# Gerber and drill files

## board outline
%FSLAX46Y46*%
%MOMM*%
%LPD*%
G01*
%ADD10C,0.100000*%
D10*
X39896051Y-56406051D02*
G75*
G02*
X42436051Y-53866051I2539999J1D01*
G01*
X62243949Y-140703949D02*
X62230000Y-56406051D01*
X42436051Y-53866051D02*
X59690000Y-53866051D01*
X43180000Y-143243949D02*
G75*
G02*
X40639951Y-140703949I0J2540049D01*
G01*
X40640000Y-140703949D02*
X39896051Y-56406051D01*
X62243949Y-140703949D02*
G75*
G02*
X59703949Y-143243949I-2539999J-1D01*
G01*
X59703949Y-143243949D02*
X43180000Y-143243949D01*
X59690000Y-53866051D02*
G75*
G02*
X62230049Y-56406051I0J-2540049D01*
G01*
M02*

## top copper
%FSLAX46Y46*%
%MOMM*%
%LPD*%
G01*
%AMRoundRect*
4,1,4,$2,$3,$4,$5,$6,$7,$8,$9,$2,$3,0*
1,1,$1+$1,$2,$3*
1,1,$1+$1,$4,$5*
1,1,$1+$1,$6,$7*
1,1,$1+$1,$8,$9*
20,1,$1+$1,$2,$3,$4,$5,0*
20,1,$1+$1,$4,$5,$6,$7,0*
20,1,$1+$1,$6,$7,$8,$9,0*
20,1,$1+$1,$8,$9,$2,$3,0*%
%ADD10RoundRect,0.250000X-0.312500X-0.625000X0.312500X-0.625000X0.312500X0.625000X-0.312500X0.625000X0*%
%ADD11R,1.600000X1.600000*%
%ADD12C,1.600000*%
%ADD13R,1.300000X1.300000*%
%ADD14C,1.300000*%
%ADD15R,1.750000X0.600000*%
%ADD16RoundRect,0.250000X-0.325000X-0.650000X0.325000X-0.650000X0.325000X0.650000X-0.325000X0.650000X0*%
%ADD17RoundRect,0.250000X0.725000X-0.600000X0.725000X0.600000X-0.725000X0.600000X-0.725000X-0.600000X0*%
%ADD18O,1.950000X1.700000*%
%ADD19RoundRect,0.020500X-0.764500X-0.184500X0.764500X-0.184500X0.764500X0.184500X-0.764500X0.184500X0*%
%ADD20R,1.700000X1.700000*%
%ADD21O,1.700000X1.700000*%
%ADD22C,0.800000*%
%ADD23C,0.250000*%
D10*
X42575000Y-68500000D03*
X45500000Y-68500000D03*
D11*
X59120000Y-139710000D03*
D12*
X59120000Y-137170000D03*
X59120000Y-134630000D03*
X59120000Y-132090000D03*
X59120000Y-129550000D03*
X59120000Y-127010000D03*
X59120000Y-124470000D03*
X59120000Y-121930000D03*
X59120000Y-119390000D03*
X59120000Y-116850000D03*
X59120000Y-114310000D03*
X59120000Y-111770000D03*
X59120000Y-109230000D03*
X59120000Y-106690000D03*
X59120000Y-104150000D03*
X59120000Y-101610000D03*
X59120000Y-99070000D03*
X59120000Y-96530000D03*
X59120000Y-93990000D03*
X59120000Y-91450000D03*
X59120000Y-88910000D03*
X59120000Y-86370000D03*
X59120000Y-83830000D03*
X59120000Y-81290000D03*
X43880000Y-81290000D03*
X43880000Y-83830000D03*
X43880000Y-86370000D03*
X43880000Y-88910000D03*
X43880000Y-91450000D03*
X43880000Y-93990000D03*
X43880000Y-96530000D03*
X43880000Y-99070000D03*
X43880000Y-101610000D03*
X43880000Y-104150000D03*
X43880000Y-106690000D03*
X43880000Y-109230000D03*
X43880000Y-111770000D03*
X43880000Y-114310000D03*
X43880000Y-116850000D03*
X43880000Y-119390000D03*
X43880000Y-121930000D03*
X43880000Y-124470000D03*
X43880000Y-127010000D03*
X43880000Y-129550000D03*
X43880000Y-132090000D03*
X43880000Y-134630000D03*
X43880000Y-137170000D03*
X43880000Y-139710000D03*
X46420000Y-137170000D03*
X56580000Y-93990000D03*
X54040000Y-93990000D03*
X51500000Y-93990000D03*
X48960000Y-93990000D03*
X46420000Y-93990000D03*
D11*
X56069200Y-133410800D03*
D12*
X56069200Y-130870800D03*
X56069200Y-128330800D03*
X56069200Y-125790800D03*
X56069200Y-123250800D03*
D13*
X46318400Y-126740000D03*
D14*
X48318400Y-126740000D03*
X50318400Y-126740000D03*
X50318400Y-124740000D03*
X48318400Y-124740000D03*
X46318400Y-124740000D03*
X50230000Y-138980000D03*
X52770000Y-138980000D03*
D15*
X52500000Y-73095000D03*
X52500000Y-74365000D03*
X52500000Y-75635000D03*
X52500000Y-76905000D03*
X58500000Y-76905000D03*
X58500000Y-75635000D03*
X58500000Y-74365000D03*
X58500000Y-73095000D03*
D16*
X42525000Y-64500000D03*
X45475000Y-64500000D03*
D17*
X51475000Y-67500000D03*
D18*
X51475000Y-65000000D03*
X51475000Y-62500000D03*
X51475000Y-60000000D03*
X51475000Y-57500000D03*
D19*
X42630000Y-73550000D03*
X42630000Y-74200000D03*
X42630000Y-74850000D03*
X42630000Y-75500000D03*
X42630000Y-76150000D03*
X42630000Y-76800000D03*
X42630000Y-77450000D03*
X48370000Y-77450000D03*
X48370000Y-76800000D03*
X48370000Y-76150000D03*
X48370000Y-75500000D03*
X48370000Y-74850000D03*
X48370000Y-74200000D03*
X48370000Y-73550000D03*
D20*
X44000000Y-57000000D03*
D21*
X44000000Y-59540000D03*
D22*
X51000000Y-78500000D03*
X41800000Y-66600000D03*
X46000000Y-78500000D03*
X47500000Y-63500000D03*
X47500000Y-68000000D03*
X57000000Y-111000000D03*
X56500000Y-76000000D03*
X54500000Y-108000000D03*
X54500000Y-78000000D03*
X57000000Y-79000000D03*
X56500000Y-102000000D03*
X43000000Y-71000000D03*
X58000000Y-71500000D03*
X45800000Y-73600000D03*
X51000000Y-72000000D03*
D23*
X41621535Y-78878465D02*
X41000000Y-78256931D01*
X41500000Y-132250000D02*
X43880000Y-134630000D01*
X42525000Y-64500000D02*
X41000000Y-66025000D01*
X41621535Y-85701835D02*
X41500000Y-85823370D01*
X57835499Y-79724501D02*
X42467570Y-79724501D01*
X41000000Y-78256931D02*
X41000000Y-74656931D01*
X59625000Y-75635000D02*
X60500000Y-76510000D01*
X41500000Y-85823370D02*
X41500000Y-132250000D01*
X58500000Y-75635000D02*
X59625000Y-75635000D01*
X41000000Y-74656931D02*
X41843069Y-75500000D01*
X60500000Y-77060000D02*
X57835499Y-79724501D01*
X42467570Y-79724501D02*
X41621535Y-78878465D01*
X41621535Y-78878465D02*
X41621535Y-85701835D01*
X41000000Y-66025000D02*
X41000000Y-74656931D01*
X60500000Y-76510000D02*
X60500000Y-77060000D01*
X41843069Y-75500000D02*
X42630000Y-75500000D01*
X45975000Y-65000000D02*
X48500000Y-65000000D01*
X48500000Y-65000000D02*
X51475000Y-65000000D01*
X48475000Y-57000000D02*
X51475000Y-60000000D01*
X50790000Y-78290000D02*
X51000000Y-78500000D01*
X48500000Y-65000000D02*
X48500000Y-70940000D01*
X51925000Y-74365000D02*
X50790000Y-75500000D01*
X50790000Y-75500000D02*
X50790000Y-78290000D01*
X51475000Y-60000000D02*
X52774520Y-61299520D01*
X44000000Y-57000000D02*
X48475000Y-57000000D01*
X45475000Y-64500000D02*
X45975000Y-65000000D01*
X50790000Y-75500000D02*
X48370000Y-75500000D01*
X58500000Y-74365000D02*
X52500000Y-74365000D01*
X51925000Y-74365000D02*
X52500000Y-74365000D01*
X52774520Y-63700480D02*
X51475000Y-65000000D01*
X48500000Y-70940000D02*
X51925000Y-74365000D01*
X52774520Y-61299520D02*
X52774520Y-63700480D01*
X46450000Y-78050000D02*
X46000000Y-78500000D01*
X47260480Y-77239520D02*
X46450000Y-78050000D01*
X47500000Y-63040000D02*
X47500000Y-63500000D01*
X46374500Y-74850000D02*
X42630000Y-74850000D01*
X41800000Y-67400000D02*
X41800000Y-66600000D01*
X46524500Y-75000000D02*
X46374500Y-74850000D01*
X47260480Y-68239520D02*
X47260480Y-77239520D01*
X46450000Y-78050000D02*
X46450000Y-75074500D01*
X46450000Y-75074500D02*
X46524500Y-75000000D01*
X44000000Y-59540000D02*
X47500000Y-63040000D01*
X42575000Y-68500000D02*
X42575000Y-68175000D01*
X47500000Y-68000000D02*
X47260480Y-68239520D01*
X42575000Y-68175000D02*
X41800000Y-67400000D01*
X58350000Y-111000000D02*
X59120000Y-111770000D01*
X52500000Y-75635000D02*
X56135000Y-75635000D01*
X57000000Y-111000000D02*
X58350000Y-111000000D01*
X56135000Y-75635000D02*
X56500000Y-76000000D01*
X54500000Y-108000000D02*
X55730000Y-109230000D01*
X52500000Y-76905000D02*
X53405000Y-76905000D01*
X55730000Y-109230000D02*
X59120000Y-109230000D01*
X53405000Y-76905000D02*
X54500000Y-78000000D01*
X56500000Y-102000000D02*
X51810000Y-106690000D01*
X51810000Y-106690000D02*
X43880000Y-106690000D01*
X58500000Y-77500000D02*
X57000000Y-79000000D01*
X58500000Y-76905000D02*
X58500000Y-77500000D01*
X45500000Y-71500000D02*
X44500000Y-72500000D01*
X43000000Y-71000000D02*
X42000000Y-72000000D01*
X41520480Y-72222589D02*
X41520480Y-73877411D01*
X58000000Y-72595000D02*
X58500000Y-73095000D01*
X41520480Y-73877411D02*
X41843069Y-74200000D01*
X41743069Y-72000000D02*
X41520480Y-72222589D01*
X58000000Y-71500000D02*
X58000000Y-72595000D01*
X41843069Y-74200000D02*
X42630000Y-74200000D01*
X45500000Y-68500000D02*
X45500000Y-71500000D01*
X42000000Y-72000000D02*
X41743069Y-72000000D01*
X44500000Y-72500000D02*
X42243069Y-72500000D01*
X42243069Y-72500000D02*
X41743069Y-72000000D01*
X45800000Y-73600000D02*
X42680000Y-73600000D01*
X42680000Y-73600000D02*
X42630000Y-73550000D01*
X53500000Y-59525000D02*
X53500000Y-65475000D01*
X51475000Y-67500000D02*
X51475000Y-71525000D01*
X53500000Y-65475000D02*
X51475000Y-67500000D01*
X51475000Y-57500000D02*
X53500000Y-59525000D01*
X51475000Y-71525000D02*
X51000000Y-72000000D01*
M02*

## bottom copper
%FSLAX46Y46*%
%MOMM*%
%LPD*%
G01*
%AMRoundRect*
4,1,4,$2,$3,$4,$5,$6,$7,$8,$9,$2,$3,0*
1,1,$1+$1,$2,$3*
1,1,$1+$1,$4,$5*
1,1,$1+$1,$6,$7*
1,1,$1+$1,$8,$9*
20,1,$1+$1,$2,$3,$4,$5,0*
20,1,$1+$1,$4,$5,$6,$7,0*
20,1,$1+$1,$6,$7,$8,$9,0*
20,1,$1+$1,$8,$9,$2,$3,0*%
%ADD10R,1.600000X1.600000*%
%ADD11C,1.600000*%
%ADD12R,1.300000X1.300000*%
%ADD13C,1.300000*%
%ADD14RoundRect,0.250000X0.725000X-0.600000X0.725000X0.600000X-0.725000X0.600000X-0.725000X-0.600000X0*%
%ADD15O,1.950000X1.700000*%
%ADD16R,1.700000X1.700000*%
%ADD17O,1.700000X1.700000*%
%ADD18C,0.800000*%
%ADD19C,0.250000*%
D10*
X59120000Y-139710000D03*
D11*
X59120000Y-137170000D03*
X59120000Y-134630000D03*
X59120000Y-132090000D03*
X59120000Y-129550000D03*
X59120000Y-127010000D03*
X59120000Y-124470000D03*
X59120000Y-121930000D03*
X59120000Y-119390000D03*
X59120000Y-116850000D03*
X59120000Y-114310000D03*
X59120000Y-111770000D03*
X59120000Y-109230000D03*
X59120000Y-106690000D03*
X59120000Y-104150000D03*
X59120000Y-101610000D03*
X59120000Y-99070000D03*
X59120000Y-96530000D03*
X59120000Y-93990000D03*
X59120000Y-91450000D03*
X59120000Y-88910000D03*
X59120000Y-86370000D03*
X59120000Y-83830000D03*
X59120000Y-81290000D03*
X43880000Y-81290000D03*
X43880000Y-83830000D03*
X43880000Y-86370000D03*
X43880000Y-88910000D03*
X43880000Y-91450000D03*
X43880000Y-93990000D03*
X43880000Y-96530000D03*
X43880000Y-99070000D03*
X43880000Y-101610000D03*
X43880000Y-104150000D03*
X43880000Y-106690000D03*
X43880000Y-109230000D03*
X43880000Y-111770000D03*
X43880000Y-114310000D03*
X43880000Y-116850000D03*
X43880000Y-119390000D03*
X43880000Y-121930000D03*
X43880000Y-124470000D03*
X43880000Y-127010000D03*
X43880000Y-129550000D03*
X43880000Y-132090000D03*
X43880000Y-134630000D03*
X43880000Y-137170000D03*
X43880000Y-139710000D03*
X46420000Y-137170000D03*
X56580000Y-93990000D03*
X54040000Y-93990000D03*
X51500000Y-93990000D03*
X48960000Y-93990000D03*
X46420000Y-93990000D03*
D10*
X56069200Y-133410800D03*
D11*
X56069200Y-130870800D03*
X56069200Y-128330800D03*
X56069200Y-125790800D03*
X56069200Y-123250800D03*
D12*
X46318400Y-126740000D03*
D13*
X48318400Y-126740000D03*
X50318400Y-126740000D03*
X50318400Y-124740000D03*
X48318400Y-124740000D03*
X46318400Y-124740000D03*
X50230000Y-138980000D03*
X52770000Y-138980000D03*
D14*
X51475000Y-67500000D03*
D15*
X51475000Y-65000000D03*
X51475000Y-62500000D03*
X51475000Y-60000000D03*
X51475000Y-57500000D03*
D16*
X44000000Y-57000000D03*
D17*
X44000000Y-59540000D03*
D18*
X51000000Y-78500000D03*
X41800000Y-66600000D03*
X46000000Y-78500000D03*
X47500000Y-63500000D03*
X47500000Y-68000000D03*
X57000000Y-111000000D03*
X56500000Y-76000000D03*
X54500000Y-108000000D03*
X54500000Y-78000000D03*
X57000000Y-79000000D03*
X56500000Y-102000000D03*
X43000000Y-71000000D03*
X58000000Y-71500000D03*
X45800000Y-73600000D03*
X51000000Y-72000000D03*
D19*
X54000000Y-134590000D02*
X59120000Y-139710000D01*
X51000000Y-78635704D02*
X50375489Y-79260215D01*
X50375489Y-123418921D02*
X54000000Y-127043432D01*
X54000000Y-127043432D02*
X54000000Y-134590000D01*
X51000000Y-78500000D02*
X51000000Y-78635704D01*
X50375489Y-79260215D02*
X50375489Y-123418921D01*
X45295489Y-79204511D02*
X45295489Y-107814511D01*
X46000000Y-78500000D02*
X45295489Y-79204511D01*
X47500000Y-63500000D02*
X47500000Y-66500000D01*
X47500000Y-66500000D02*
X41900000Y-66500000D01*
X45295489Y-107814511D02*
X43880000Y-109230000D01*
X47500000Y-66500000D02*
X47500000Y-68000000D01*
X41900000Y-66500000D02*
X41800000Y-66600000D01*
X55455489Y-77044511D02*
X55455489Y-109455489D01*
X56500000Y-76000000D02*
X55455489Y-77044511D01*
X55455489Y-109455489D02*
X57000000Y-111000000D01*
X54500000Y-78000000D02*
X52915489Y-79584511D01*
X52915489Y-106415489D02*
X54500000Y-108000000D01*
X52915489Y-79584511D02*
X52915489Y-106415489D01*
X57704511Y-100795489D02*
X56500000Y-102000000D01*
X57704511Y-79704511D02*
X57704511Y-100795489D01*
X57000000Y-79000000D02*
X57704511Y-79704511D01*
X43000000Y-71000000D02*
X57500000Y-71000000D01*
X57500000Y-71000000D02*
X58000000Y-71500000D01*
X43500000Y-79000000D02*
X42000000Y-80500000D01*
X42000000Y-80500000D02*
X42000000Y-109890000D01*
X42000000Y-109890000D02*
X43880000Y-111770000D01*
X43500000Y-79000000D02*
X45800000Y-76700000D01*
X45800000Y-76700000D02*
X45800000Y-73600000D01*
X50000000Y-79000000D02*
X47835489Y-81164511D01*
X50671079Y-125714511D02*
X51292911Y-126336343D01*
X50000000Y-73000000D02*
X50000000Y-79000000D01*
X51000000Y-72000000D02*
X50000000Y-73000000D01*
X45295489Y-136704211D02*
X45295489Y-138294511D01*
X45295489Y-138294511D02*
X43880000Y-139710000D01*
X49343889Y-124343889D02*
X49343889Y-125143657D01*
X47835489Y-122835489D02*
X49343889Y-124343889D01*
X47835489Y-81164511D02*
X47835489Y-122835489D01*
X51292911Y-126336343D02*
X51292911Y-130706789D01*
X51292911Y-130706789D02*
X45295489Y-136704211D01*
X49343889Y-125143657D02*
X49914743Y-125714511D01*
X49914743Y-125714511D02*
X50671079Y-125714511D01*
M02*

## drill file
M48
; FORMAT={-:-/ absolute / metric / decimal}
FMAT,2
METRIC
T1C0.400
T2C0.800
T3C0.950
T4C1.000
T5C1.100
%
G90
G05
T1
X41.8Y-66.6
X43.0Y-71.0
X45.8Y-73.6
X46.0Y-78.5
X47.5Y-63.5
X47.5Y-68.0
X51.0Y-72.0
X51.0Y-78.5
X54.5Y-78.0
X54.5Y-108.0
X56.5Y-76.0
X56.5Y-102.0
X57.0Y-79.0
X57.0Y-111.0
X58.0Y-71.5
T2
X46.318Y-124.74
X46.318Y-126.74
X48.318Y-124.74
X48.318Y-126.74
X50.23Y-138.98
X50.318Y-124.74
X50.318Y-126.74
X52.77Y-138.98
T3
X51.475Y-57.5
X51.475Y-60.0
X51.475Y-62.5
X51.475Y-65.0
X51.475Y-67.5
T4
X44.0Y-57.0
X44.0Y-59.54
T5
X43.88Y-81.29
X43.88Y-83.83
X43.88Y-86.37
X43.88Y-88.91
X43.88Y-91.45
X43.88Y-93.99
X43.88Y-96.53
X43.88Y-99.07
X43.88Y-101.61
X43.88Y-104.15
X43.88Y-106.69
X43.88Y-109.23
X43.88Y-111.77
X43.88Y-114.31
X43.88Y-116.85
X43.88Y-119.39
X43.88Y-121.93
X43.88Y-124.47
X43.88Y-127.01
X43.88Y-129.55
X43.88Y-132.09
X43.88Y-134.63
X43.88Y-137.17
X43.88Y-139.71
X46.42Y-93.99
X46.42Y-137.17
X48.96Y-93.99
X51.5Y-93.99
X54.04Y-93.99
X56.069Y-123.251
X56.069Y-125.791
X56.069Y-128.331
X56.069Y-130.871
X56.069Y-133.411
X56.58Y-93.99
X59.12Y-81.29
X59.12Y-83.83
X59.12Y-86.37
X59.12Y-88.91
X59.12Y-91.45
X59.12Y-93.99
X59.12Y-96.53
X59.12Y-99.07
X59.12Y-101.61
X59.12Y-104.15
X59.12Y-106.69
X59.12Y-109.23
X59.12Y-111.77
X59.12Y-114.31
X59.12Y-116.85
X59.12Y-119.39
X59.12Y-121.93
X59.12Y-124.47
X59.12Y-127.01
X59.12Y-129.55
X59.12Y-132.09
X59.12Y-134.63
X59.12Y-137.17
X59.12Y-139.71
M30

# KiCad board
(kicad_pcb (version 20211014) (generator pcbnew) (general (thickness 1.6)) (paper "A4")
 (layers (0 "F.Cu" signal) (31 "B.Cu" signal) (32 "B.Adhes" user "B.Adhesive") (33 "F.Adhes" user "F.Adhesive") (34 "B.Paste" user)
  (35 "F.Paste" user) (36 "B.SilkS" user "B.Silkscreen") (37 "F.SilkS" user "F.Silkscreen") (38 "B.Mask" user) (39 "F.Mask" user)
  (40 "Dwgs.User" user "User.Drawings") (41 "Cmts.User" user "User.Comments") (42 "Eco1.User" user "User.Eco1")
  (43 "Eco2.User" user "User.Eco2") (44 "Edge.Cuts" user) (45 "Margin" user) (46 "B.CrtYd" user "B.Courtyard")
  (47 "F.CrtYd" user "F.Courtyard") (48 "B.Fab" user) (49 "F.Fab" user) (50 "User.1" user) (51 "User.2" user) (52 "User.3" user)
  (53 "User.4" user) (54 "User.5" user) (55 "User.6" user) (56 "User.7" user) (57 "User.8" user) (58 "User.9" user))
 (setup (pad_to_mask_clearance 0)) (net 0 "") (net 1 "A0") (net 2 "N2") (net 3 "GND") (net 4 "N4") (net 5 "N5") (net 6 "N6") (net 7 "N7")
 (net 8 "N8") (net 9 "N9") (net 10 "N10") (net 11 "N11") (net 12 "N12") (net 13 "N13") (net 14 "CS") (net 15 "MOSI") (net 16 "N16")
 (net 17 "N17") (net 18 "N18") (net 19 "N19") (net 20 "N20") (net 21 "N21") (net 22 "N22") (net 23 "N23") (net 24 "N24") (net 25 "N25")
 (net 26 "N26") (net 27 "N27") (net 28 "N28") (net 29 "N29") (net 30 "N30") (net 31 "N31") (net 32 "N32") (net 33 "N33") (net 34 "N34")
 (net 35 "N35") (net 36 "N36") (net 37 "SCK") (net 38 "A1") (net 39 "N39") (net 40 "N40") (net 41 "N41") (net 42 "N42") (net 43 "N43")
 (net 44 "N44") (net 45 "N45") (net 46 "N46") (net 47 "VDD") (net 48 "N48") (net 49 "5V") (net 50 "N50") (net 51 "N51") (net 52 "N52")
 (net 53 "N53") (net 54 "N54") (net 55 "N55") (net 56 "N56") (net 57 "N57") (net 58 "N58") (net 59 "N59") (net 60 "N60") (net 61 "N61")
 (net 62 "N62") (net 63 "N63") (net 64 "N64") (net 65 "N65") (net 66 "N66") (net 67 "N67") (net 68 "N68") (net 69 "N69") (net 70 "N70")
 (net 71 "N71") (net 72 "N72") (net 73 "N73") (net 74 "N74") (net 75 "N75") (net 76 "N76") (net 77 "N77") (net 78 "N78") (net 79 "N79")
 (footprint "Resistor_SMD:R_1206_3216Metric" (layer "F.Cu") (at 44.0375 68.5)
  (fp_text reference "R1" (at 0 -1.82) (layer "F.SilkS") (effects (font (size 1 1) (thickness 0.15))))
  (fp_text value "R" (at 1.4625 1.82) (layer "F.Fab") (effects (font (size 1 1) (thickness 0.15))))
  (pad "1" smd roundrect (at -1.4625 0) (size 1.125 1.75) (layers "F.Cu" "F.Paste" "F.Mask") (roundrect_rratio 0.2222222222) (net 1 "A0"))
  (pad "2" smd roundrect (at 1.4625 0) (size 1.125 1.75) (layers "F.Cu" "F.Paste" "F.Mask") (roundrect_rratio 0.2222222222) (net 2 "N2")))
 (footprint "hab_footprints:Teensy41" (layer "F.Cu") (at 51.5 110.5 90)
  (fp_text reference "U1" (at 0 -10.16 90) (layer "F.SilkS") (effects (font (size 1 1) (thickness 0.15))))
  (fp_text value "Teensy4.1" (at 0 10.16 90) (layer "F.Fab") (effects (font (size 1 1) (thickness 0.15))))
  (pad "1" thru_hole rect locked (at -29.21 7.62 90) (size 1.6 1.6) (drill 1.1) (layers *.Cu *.Mask) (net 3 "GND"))
  (pad "2" thru_hole circle locked (at -26.67 7.62 90) (size 1.6 1.6) (drill 1.1) (layers *.Cu *.Mask) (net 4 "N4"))
  (pad "3" thru_hole circle locked (at -24.13 7.62 90) (size 1.6 1.6) (drill 1.1) (layers *.Cu *.Mask) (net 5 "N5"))
  (pad "4" thru_hole circle locked (at -21.59 7.62 90) (size 1.6 1.6) (drill 1.1) (layers *.Cu *.Mask) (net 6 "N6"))
  (pad "5" thru_hole circle locked (at -19.05 7.62 90) (size 1.6 1.6) (drill 1.1) (layers *.Cu *.Mask) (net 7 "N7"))
  (pad "6" thru_hole circle locked (at -16.51 7.62 90) (size 1.6 1.6) (drill 1.1) (layers *.Cu *.Mask) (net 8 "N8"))
  (pad "7" thru_hole circle locked (at -13.97 7.62 90) (size 1.6 1.6) (drill 1.1) (layers *.Cu *.Mask) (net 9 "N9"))
  (pad "8" thru_hole circle locked (at -11.43 7.62 90) (size 1.6 1.6) (drill 1.1) (layers *.Cu *.Mask) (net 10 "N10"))
  (pad "9" thru_hole circle locked (at -8.89 7.62 90) (size 1.6 1.6) (drill 1.1) (layers *.Cu *.Mask) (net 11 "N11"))
  (pad "10" thru_hole circle locked (at -6.35 7.62 90) (size 1.6 1.6) (drill 1.1) (layers *.Cu *.Mask) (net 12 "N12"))
  (pad "11" thru_hole circle locked (at -3.81 7.62 90) (size 1.6 1.6) (drill 1.1) (layers *.Cu *.Mask) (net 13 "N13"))
  (pad "12" thru_hole circle locked (at -1.27 7.62 90) (size 1.6 1.6) (drill 1.1) (layers *.Cu *.Mask) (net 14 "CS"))
  (pad "13" thru_hole circle locked (at 1.27 7.62 90) (size 1.6 1.6) (drill 1.1) (layers *.Cu *.Mask) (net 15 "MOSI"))
  (pad "14" thru_hole circle locked (at 3.81 7.62 90) (size 1.6 1.6) (drill 1.1) (layers *.Cu *.Mask) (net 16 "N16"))
  (pad "15" thru_hole circle locked (at 6.35 7.62 90) (size 1.6 1.6) (drill 1.1) (layers *.Cu *.Mask) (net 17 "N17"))
  (pad "16" thru_hole circle locked (at 8.89 7.62 90) (size 1.6 1.6) (drill 1.1) (layers *.Cu *.Mask) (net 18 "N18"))
  (pad "17" thru_hole circle locked (at 11.43 7.62 90) (size 1.6 1.6) (drill 1.1) (layers *.Cu *.Mask) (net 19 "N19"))
  (pad "18" thru_hole circle locked (at 13.97 7.62 90) (size 1.6 1.6) (drill 1.1) (layers *.Cu *.Mask) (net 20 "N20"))
  (pad "19" thru_hole circle locked (at 16.51 7.62 90) (size 1.6 1.6) (drill 1.1) (layers *.Cu *.Mask) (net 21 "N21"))
  (pad "20" thru_hole circle locked (at 19.05 7.62 90) (size 1.6 1.6) (drill 1.1) (layers *.Cu *.Mask) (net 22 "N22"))
  (pad "21" thru_hole circle locked (at 21.59 7.62 90) (size 1.6 1.6) (drill 1.1) (layers *.Cu *.Mask) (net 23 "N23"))
  (pad "22" thru_hole circle locked (at 24.13 7.62 90) (size 1.6 1.6) (drill 1.1) (layers *.Cu *.Mask) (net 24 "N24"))
  (pad "23" thru_hole circle locked (at 26.67 7.62 90) (size 1.6 1.6) (drill 1.1) (layers *.Cu *.Mask) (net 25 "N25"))
  (pad "24" thru_hole circle locked (at 29.21 7.62 90) (size 1.6 1.6) (drill 1.1) (layers *.Cu *.Mask) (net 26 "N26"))
  (pad "25" thru_hole circle locked (at 29.21 -7.62 90) (size 1.6 1.6) (drill 1.1) (layers *.Cu *.Mask) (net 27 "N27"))
  (pad "26" thru_hole circle locked (at 26.67 -7.62 90) (size 1.6 1.6) (drill 1.1) (layers *.Cu *.Mask) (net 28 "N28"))
  (pad "27" thru_hole circle locked (at 24.13 -7.62 90) (size 1.6 1.6) (drill 1.1) (layers *.Cu *.Mask) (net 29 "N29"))
  (pad "28" thru_hole circle locked (at 21.59 -7.62 90) (size 1.6 1.6) (drill 1.1) (layers *.Cu *.Mask) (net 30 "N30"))
  (pad "29" thru_hole circle locked (at 19.05 -7.62 90) (size 1.6 1.6) (drill 1.1) (layers *.Cu *.Mask) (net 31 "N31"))
  (pad "30" thru_hole circle locked (at 16.51 -7.62 90) (size 1.6 1.6) (drill 1.1) (layers *.Cu *.Mask) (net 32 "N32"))
  (pad "31" thru_hole circle locked (at 13.97 -7.62 90) (size 1.6 1.6) (drill 1.1) (layers *.Cu *.Mask) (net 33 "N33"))
  (pad "32" thru_hole circle locked (at 11.43 -7.62 90) (size 1.6 1.6) (drill 1.1) (layers *.Cu *.Mask) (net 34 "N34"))
  (pad "33" thru_hole circle locked (at 8.89 -7.62 90) (size 1.6 1.6) (drill 1.1) (layers *.Cu *.Mask) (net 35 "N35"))
  (pad "34" thru_hole circle locked (at 6.35 -7.62 90) (size 1.6 1.6) (drill 1.1) (layers *.Cu *.Mask) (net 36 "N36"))
  (pad "35" thru_hole circle locked (at 3.81 -7.62 90) (size 1.6 1.6) (drill 1.1) (layers *.Cu *.Mask) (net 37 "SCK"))
  (pad "36" thru_hole circle locked (at 1.27 -7.62 90) (size 1.6 1.6) (drill 1.1) (layers *.Cu *.Mask) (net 1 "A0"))
  (pad "37" thru_hole circle locked (at -1.27 -7.62 90) (size 1.6 1.6) (drill 1.1) (layers *.Cu *.Mask) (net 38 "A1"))
  (pad "38" thru_hole circle locked (at -3.81 -7.62 90) (size 1.6 1.6) (drill 1.1) (layers *.Cu *.Mask) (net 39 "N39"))
  (pad "39" thru_hole circle locked (at -6.35 -7.62 90) (size 1.6 1.6) (drill 1.1) (layers *.Cu *.Mask) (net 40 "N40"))
  (pad "40" thru_hole circle locked (at -8.89 -7.62 90) (size 1.6 1.6) (drill 1.1) (layers *.Cu *.Mask) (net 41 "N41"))
  (pad "41" thru_hole circle locked (at -11.43 -7.62 90) (size 1.6 1.6) (drill 1.1) (layers *.Cu *.Mask) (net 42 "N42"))
  (pad "42" thru_hole circle locked (at -13.97 -7.62 90) (size 1.6 1.6) (drill 1.1) (layers *.Cu *.Mask) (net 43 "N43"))
  (pad "43" thru_hole circle locked (at -16.51 -7.62 90) (size 1.6 1.6) (drill 1.1) (layers *.Cu *.Mask) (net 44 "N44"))
  (pad "44" thru_hole circle locked (at -19.05 -7.62 90) (size 1.6 1.6) (drill 1.1) (layers *.Cu *.Mask) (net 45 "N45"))
  (pad "45" thru_hole circle locked (at -21.59 -7.62 90) (size 1.6 1.6) (drill 1.1) (layers *.Cu *.Mask) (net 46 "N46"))
  (pad "46" thru_hole circle locked (at -24.13 -7.62 90) (size 1.6 1.6) (drill 1.1) (layers *.Cu *.Mask) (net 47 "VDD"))
  (pad "47" thru_hole circle locked (at -26.67 -7.62 90) (size 1.6 1.6) (drill 1.1) (layers *.Cu *.Mask) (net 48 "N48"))
  (pad "48" thru_hole circle locked (at -29.21 -7.62 90) (size 1.6 1.6) (drill 1.1) (layers *.Cu *.Mask) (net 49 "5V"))
  (pad "49" thru_hole circle locked (at -26.67 -5.08 90) (size 1.6 1.6) (drill 1.1) (layers *.Cu *.Mask) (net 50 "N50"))
  (pad "50" thru_hole circle locked (at 16.51 5.08 90) (size 1.6 1.6) (drill 1.1) (layers *.Cu *.Mask) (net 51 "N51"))
  (pad "51" thru_hole circle locked (at 16.51 2.54 90) (size 1.6 1.6) (drill 1.1) (layers *.Cu *.Mask) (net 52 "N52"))
  (pad "52" thru_hole circle locked (at 16.51 0 90) (size 1.6 1.6) (drill 1.1) (layers *.Cu *.Mask) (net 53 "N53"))
  (pad "53" thru_hole circle locked (at 16.51 -2.54 90) (size 1.6 1.6) (drill 1.1) (layers *.Cu *.Mask) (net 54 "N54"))
  (pad "54" thru_hole circle locked (at 16.51 -5.08 90) (size 1.6 1.6) (drill 1.1) (layers *.Cu *.Mask) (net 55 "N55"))
  (pad "55" thru_hole rect locked (at -22.9108 4.5692 90) (size 1.6 1.6) (drill 1.1) (layers *.Cu *.Mask) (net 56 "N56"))
  (pad "56" thru_hole circle locked (at -20.3708 4.5692 90) (size 1.6 1.6) (drill 1.1) (layers *.Cu *.Mask) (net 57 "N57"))
  (pad "57" thru_hole circle locked (at -17.8308 4.5692 90) (size 1.6 1.6) (drill 1.1) (layers *.Cu *.Mask) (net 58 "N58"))
  (pad "58" thru_hole circle locked (at -15.2908 4.5692 90) (size 1.6 1.6) (drill 1.1) (layers *.Cu *.Mask) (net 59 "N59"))
  (pad "59" thru_hole circle locked (at -12.7508 4.5692 90) (size 1.6 1.6) (drill 1.1) (layers *.Cu *.Mask) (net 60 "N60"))
  (pad "60" thru_hole rect locked (at -16.24 -5.1816 90) (size 1.3 1.3) (drill 0.8) (layers *.Cu *.Mask) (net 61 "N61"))
  (pad "61" thru_hole circle locked (at -16.24 -3.1816 90) (size 1.3 1.3) (drill 0.8) (layers *.Cu *.Mask) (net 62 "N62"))
  (pad "62" thru_hole circle locked (at -16.24 -1.1816 90) (size 1.3 1.3) (drill 0.8) (layers *.Cu *.Mask) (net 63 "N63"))
  (pad "63" thru_hole circle locked (at -14.24 -1.1816 90) (size 1.3 1.3) (drill 0.8) (layers *.Cu *.Mask) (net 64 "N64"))
  (pad "64" thru_hole circle locked (at -14.24 -3.1816 90) (size 1.3 1.3) (drill 0.8) (layers *.Cu *.Mask) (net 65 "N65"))
  (pad "65" thru_hole circle locked (at -14.24 -5.1816 90) (size 1.3 1.3) (drill 0.8) (layers *.Cu *.Mask) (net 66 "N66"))
  (pad "66" thru_hole circle locked (at -28.48 -1.27 90) (size 1.3 1.3) (drill 0.8) (layers *.Cu *.Mask) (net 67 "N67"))
  (pad "67" thru_hole circle locked (at -28.48 1.27 90) (size 1.3 1.3) (drill 0.8) (layers *.Cu *.Mask) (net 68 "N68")))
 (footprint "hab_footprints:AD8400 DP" (layer "F.Cu") (at 55.5 75 -90)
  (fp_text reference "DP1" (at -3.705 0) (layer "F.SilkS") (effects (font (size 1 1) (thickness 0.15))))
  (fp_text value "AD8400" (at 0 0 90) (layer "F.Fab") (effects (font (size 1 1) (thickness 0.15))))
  (pad "1" smd rect (at -1.905 3 270) (size 0.6 1.75) (layers "F.Cu" "F.Paste" "F.Mask") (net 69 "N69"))
  (pad "2" smd rect (at -0.635 3 270) (size 0.6 1.75) (layers "F.Cu" "F.Paste" "F.Mask") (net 3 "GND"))
  (pad "3" smd rect (at 0.635 3 270) (size 0.6 1.75) (layers "F.Cu" "F.Paste" "F.Mask") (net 14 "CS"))
  (pad "4" smd rect (at 1.905 3 270) (size 0.6 1.75) (layers "F.Cu" "F.Paste" "F.Mask") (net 15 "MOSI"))
  (pad "5" smd rect (at 1.905 -3 270) (size 0.6 1.75) (layers "F.Cu" "F.Paste" "F.Mask") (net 37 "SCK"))
  (pad "6" smd rect (at 0.635 -3 270) (size 0.6 1.75) (layers "F.Cu" "F.Paste" "F.Mask") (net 47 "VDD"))
  (pad "7" smd rect (at -0.635 -3 270) (size 0.6 1.75) (layers "F.Cu" "F.Paste" "F.Mask") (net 3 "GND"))
  (pad "8" smd rect (at -1.905 -3 270) (size 0.6 1.75) (layers "F.Cu" "F.Paste" "F.Mask") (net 2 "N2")))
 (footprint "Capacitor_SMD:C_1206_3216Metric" (layer "F.Cu") (at 44 64.5)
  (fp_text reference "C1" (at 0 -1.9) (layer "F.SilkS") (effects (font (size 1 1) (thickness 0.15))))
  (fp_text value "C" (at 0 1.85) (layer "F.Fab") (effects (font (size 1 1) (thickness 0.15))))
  (pad "1" smd roundrect (at -1.475 0) (size 1.15 1.8) (layers "F.Cu" "F.Paste" "F.Mask") (roundrect_rratio 0.2173913043) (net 47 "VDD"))
  (pad "2" smd roundrect (at 1.475 0) (size 1.15 1.8) (layers "F.Cu" "F.Paste" "F.Mask") (roundrect_rratio 0.2173913043) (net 3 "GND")))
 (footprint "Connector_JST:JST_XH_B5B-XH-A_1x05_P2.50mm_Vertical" (layer "F.Cu") (at 51.475 67.5 90)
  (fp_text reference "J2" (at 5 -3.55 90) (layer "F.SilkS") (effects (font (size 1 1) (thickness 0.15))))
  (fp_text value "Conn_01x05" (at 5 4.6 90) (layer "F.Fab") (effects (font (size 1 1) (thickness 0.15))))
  (pad "1" thru_hole roundrect (at 0 0 90) (size 1.7 1.95) (drill 0.95) (layers *.Cu *.Mask) (roundrect_rratio 0.1470588235) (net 49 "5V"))
  (pad "2" thru_hole oval (at 2.5 0 90) (size 1.7 1.95) (drill 0.95) (layers *.Cu *.Mask) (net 3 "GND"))
  (pad "3" thru_hole oval (at 5 0 90) (size 1.7 1.95) (drill 0.95) (layers *.Cu *.Mask) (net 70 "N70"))
  (pad "4" thru_hole oval (at 7.5 0 90) (size 1.7 1.95) (drill 0.95) (layers *.Cu *.Mask) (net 3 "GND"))
  (pad "5" thru_hole oval (at 10 0 90) (size 1.7 1.95) (drill 0.95) (layers *.Cu *.Mask) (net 49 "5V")))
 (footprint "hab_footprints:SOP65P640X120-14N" (layer "F.Cu") (at 45.5 75.5)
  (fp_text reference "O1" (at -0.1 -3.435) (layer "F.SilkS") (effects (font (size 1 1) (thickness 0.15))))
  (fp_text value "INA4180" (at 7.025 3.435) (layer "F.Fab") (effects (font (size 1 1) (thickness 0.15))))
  (pad "1" smd roundrect locked (at -2.87 -1.95) (size 1.57 0.41) (layers "F.Cu" "F.Paste" "F.Mask") (roundrect_rratio 0.05) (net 38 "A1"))
  (pad "2" smd roundrect locked (at -2.87 -1.3) (size 1.57 0.41) (layers "F.Cu" "F.Paste" "F.Mask") (roundrect_rratio 0.05) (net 2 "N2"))
  (pad "3" smd roundrect locked (at -2.87 -0.65) (size 1.57 0.41) (layers "F.Cu" "F.Paste" "F.Mask") (roundrect_rratio 0.05) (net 1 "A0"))
  (pad "4" smd roundrect locked (at -2.87 0) (size 1.57 0.41) (layers "F.Cu" "F.Paste" "F.Mask") (roundrect_rratio 0.05) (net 47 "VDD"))
  (pad "5" smd roundrect locked (at -2.87 0.65) (size 1.57 0.41) (layers "F.Cu" "F.Paste" "F.Mask") (roundrect_rratio 0.05) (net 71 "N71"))
  (pad "6" smd roundrect locked (at -2.87 1.3) (size 1.57 0.41) (layers "F.Cu" "F.Paste" "F.Mask") (roundrect_rratio 0.05) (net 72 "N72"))
  (pad "7" smd roundrect locked (at -2.87 1.95) (size 1.57 0.41) (layers "F.Cu" "F.Paste" "F.Mask") (roundrect_rratio 0.05) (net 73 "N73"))
  (pad "8" smd roundrect locked (at 2.87 1.95) (size 1.57 0.41) (layers "F.Cu" "F.Paste" "F.Mask") (roundrect_rratio 0.05) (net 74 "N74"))
  (pad "9" smd roundrect locked (at 2.87 1.3) (size 1.57 0.41) (layers "F.Cu" "F.Paste" "F.Mask") (roundrect_rratio 0.05) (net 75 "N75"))
  (pad "10" smd roundrect locked (at 2.87 0.65) (size 1.57 0.41) (layers "F.Cu" "F.Paste" "F.Mask") (roundrect_rratio 0.05) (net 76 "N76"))
  (pad "11" smd roundrect locked (at 2.87 0) (size 1.57 0.41) (layers "F.Cu" "F.Paste" "F.Mask") (roundrect_rratio 0.05) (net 3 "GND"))
  (pad "12" smd roundrect locked (at 2.87 -0.65) (size 1.57 0.41) (layers "F.Cu" "F.Paste" "F.Mask") (roundrect_rratio 0.05) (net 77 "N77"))
  (pad "13" smd roundrect locked (at 2.87 -1.3) (size 1.57 0.41) (layers "F.Cu" "F.Paste" "F.Mask") (roundrect_rratio 0.05) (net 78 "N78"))
  (pad "14" smd roundrect locked (at 2.87 -1.95) (size 1.57 0.41) (layers "F.Cu" "F.Paste" "F.Mask") (roundrect_rratio 0.05) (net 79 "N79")))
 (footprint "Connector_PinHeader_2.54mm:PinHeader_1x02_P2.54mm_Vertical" (layer "F.Cu") (at 44 57)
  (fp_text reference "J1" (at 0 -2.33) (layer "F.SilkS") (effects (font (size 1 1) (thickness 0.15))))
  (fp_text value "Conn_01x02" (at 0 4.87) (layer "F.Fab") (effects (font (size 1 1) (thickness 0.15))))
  (pad "1" thru_hole rect (at 0 0) (size 1.7 1.7) (drill 1) (layers *.Cu *.Mask) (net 3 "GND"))
  (pad "2" thru_hole oval (at 0 2.54) (size 1.7 1.7) (drill 1) (layers *.Cu *.Mask) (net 1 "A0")))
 (gr_arc (start 39.896051 56.406051) (mid 40.64 54.61) (end 42.436051 53.866051) (layer "Edge.Cuts") (width 0.1))
 (gr_line (start 62.243949 140.703949) (end 62.23 56.406051) (layer "Edge.Cuts") (width 0.1))
 (gr_line (start 42.436051 53.866051) (end 59.69 53.866051) (layer "Edge.Cuts") (width 0.1))
 (gr_arc (start 43.18 143.243949) (mid 41.383949 142.5) (end 40.64 140.703949) (layer "Edge.Cuts") (width 0.1))
 (gr_line (start 40.64 140.703949) (end 39.896051 56.406051) (layer "Edge.Cuts") (width 0.1))
 (gr_arc (start 62.243949 140.703949) (mid 61.5 142.5) (end 59.703949 143.243949) (layer "Edge.Cuts") (width 0.1))
 (gr_line (start 59.703949 143.243949) (end 43.18 143.243949) (layer "Edge.Cuts") (width 0.1))
 (gr_arc (start 59.69 53.866051) (mid 61.486051 54.61) (end 62.23 56.406051) (layer "Edge.Cuts") (width 0.1))
 (segment (start 41.621535 78.878465) (end 41 78.256931) (width 0.25) (layer "F.Cu") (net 47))
 (segment (start 41.5 132.25) (end 43.88 134.63) (width 0.25) (layer "F.Cu") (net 47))
 (segment (start 42.525 64.5) (end 41 66.025) (width 0.25) (layer "F.Cu") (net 47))
 (segment (start 41.621535 85.701835) (end 41.5 85.82337) (width 0.25) (layer "F.Cu") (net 47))
 (segment (start 57.835499 79.724501) (end 42.46757 79.724501) (width 0.25) (layer "F.Cu") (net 47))
 (segment (start 41 78.256931) (end 41 74.656931) (width 0.25) (layer "F.Cu") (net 47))
 (segment (start 59.625 75.635) (end 60.5 76.51) (width 0.25) (layer "F.Cu") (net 47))
 (segment (start 41.5 85.82337) (end 41.5 132.25) (width 0.25) (layer "F.Cu") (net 47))
 (segment (start 58.5 75.635) (end 59.625 75.635) (width 0.25) (layer "F.Cu") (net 47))
 (segment (start 41 74.656931) (end 41.843069 75.5) (width 0.25) (layer "F.Cu") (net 47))
 (segment (start 60.5 77.06) (end 57.835499 79.724501) (width 0.25) (layer "F.Cu") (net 47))
 (segment (start 42.46757 79.724501) (end 41.621535 78.878465) (width 0.25) (layer "F.Cu") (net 47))
 (segment (start 41.621535 78.878465) (end 41.621535 85.701835) (width 0.25) (layer "F.Cu") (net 47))
 (segment (start 41 66.025) (end 41 74.656931) (width 0.25) (layer "F.Cu") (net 47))
 (segment (start 60.5 76.51) (end 60.5 77.06) (width 0.25) (layer "F.Cu") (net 47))
 (segment (start 41.843069 75.5) (end 42.63 75.5) (width 0.25) (layer "F.Cu") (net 47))
 (segment (start 45.975 65) (end 48.5 65) (width 0.25) (layer "F.Cu") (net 3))
 (segment (start 48.5 65) (end 51.475 65) (width 0.25) (layer "F.Cu") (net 3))
 (segment (start 48.475 57) (end 51.475 60) (width 0.25) (layer "F.Cu") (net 3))
 (segment (start 50.79 78.29) (end 51 78.5) (width 0.25) (layer "F.Cu") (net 3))
 (segment (start 48.5 65) (end 48.5 70.94) (width 0.25) (layer "F.Cu") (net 3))
 (segment (start 51.925 74.365) (end 50.79 75.5) (width 0.25) (layer "F.Cu") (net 3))
 (segment (start 50.79 75.5) (end 50.79 78.29) (width 0.25) (layer "F.Cu") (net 3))
 (segment (start 51.475 60) (end 52.77452 61.29952) (width 0.25) (layer "F.Cu") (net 3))
 (segment (start 44 57) (end 48.475 57) (width 0.25) (layer "F.Cu") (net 3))
 (segment (start 45.475 64.5) (end 45.975 65) (width 0.25) (layer "F.Cu") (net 3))
 (segment (start 50.79 75.5) (end 48.37 75.5) (width 0.25) (layer "F.Cu") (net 3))
 (segment (start 58.5 74.365) (end 52.5 74.365) (width 0.25) (layer "F.Cu") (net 3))
 (segment (start 51.925 74.365) (end 52.5 74.365) (width 0.25) (layer "F.Cu") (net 3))
 (segment (start 52.77452 63.70048) (end 51.475 65) (width 0.25) (layer "F.Cu") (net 3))
 (segment (start 48.5 70.94) (end 51.925 74.365) (width 0.25) (layer "F.Cu") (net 3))
 (segment (start 52.77452 61.29952) (end 52.77452 63.70048) (width 0.25) (layer "F.Cu") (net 3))
 (via (at 51 78.5) (size 0.8) (drill 0.4) (layers "F.Cu" "B.Cu") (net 3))
 (segment (start 54 134.59) (end 59.12 139.71) (width 0.25) (layer "B.Cu") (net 3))
 (segment (start 51 78.635704) (end 50.375489 79.260215) (width 0.25) (layer "B.Cu") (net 3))
 (segment (start 50.375489 123.418921) (end 54 127.043432) (width 0.25) (layer "B.Cu") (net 3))
 (segment (start 54 127.043432) (end 54 134.59) (width 0.25) (layer "B.Cu") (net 3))
 (segment (start 51 78.5) (end 51 78.635704) (width 0.25) (layer "B.Cu") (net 3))
 (segment (start 50.375489 79.260215) (end 50.375489 123.418921) (width 0.25) (layer "B.Cu") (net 3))
 (segment (start 46.45 78.05) (end 46 78.5) (width 0.25) (layer "F.Cu") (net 1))
 (segment (start 47.26048 77.23952) (end 46.45 78.05) (width 0.25) (layer "F.Cu") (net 1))
 (segment (start 47.5 63.04) (end 47.5 63.5) (width 0.25) (layer "F.Cu") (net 1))
 (segment (start 46.3745 74.85) (end 42.63 74.85) (width 0.25) (layer "F.Cu") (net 1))
 (segment (start 41.8 67.4) (end 41.8 66.6) (width 0.25) (layer "F.Cu") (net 1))
 (segment (start 46.5245 75) (end 46.3745 74.85) (width 0.25) (layer "F.Cu") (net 1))
 (segment (start 47.26048 68.23952) (end 47.26048 77.23952) (width 0.25) (layer "F.Cu") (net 1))
 (segment (start 46.45 78.05) (end 46.45 75.0745) (width 0.25) (layer "F.Cu") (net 1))
 (segment (start 46.45 75.0745) (end 46.5245 75) (width 0.25) (layer "F.Cu") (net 1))
 (segment (start 44 59.54) (end 47.5 63.04) (width 0.25) (layer "F.Cu") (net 1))
 (segment (start 42.575 68.5) (end 42.575 68.175) (width 0.25) (layer "F.Cu") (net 1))
 (segment (start 47.5 68) (end 47.26048 68.23952) (width 0.25) (layer "F.Cu") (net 1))
 (segment (start 42.575 68.175) (end 41.8 67.4) (width 0.25) (layer "F.Cu") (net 1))
 (via (at 41.8 66.6) (size 0.8) (drill 0.4) (layers "F.Cu" "B.Cu") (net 1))
 (via (at 46 78.5) (size 0.8) (drill 0.4) (layers "F.Cu" "B.Cu") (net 1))
 (via (at 47.5 63.5) (size 0.8) (drill 0.4) (layers "F.Cu" "B.Cu") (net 1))
 (via (at 47.5 68) (size 0.8) (drill 0.4) (layers "F.Cu" "B.Cu") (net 1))
 (segment (start 45.295489 79.204511) (end 45.295489 107.814511) (width 0.25) (layer "B.Cu") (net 1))
 (segment (start 46 78.5) (end 45.295489 79.204511) (width 0.25) (layer "B.Cu") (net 1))
 (segment (start 47.5 63.5) (end 47.5 66.5) (width 0.25) (layer "B.Cu") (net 1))
 (segment (start 47.5 66.5) (end 41.9 66.5) (width 0.25) (layer "B.Cu") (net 1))
 (segment (start 45.295489 107.814511) (end 43.88 109.23) (width 0.25) (layer "B.Cu") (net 1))
 (segment (start 47.5 66.5) (end 47.5 68) (width 0.25) (layer "B.Cu") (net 1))
 (segment (start 41.9 66.5) (end 41.8 66.6) (width 0.25) (layer "B.Cu") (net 1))
 (segment (start 58.35 111) (end 59.12 111.77) (width 0.25) (layer "F.Cu") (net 14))
 (segment (start 52.5 75.635) (end 56.135 75.635) (width 0.25) (layer "F.Cu") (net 14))
 (segment (start 57 111) (end 58.35 111) (width 0.25) (layer "F.Cu") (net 14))
 (segment (start 56.135 75.635) (end 56.5 76) (width 0.25) (layer "F.Cu") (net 14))
 (via (at 57 111) (size 0.8) (drill 0.4) (layers "F.Cu" "B.Cu") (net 14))
 (via (at 56.5 76) (size 0.8) (drill 0.4) (layers "F.Cu" "B.Cu") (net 14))
 (segment (start 55.455489 77.044511) (end 55.455489 109.455489) (width 0.25) (layer "B.Cu") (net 14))
 (segment (start 56.5 76) (end 55.455489 77.044511) (width 0.25) (layer "B.Cu") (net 14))
 (segment (start 55.455489 109.455489) (end 57 111) (width 0.25) (layer "B.Cu") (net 14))
 (segment (start 54.5 108) (end 55.73 109.23) (width 0.25) (layer "F.Cu") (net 15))
 (segment (start 52.5 76.905) (end 53.405 76.905) (width 0.25) (layer "F.Cu") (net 15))
 (segment (start 55.73 109.23) (end 59.12 109.23) (width 0.25) (layer "F.Cu") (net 15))
 (segment (start 53.405 76.905) (end 54.5 78) (width 0.25) (layer "F.Cu") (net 15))
 (via (at 54.5 108) (size 0.8) (drill 0.4) (layers "F.Cu" "B.Cu") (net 15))
 (via (at 54.5 78) (size 0.8) (drill 0.4) (layers "F.Cu" "B.Cu") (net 15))
 (segment (start 54.5 78) (end 52.915489 79.584511) (width 0.25) (layer "B.Cu") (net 15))
 (segment (start 52.915489 106.415489) (end 54.5 108) (width 0.25) (layer "B.Cu") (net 15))
 (segment (start 52.915489 79.584511) (end 52.915489 106.415489) (width 0.25) (layer "B.Cu") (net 15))
 (segment (start 56.5 102) (end 51.81 106.69) (width 0.25) (layer "F.Cu") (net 37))
 (segment (start 51.81 106.69) (end 43.88 106.69) (width 0.25) (layer "F.Cu") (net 37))
 (segment (start 58.5 77.5) (end 57 79) (width 0.25) (layer "F.Cu") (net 37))
 (segment (start 58.5 76.905) (end 58.5 77.5) (width 0.25) (layer "F.Cu") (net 37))
 (via (at 57 79) (size 0.8) (drill 0.4) (layers "F.Cu" "B.Cu") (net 37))
 (via (at 56.5 102) (size 0.8) (drill 0.4) (layers "F.Cu" "B.Cu") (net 37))
 (segment (start 57.704511 100.795489) (end 56.5 102) (width 0.25) (layer "B.Cu") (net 37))
 (segment (start 57.704511 79.704511) (end 57.704511 100.795489) (width 0.25) (layer "B.Cu") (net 37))
 (segment (start 57 79) (end 57.704511 79.704511) (width 0.25) (layer "B.Cu") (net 37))
 (segment (start 45.5 71.5) (end 44.5 72.5) (width 0.25) (layer "F.Cu") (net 2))
 (segment (start 43 71) (end 42 72) (width 0.25) (layer "F.Cu") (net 2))
 (segment (start 41.52048 72.222589) (end 41.52048 73.877411) (width 0.25) (layer "F.Cu") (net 2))
 (segment (start 58 72.595) (end 58.5 73.095) (width 0.25) (layer "F.Cu") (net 2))
 (segment (start 41.52048 73.877411) (end 41.843069 74.2) (width 0.25) (layer "F.Cu") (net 2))
 (segment (start 41.743069 72) (end 41.52048 72.222589) (width 0.25) (layer "F.Cu") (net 2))
 (segment (start 58 71.5) (end 58 72.595) (width 0.25) (layer "F.Cu") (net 2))
 (segment (start 41.843069 74.2) (end 42.63 74.2) (width 0.25) (layer "F.Cu") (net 2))
 (segment (start 45.5 68.5) (end 45.5 71.5) (width 0.25) (layer "F.Cu") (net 2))
 (segment (start 42 72) (end 41.743069 72) (width 0.25) (layer "F.Cu") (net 2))
 (segment (start 44.5 72.5) (end 42.243069 72.5) (width 0.25) (layer "F.Cu") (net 2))
 (segment (start 42.243069 72.5) (end 41.743069 72) (width 0.25) (layer "F.Cu") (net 2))
 (via (at 43 71) (size 0.8) (drill 0.4) (layers "F.Cu" "B.Cu") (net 2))
 (via (at 58 71.5) (size 0.8) (drill 0.4) (layers "F.Cu" "B.Cu") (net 2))
 (segment (start 43 71) (end 57.5 71) (width 0.25) (layer "B.Cu") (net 2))
 (segment (start 57.5 71) (end 58 71.5) (width 0.25) (layer "B.Cu") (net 2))
 (segment (start 45.8 73.6) (end 42.68 73.6) (width 0.25) (layer "F.Cu") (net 38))
 (segment (start 42.68 73.6) (end 42.63 73.55) (width 0.25) (layer "F.Cu") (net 38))
 (via (at 45.8 73.6) (size 0.8) (drill 0.4) (layers "F.Cu" "B.Cu") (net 38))
 (segment (start 43.5 79) (end 42 80.5) (width 0.25) (layer "B.Cu") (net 38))
 (segment (start 42 80.5) (end 42 109.89) (width 0.25) (layer "B.Cu") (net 38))
 (segment (start 42 109.89) (end 43.88 111.77) (width 0.25) (layer "B.Cu") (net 38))
 (segment (start 43.5 79) (end 45.8 76.7) (width 0.25) (layer "B.Cu") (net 38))
 (segment (start 45.8 76.7) (end 45.8 73.6) (width 0.25) (layer "B.Cu") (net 38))
 (segment (start 53.5 59.525) (end 53.5 65.475) (width 0.25) (layer "F.Cu") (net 49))
 (segment (start 51.475 67.5) (end 51.475 71.525) (width 0.25) (layer "F.Cu") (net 49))
 (segment (start 53.5 65.475) (end 51.475 67.5) (width 0.25) (layer "F.Cu") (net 49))
 (segment (start 51.475 57.5) (end 53.5 59.525) (width 0.25) (layer "F.Cu") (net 49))
 (segment (start 51.475 71.525) (end 51 72) (width 0.25) (layer "F.Cu") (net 49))
 (via (at 51 72) (size 0.8) (drill 0.4) (layers "F.Cu" "B.Cu") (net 49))
 (segment (start 50 79) (end 47.835489 81.164511) (width 0.25) (layer "B.Cu") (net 49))
 (segment (start 50.671079 125.714511) (end 51.292911 126.336343) (width 0.25) (layer "B.Cu") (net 49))
 (segment (start 50 73) (end 50 79) (width 0.25) (layer "B.Cu") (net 49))
 (segment (start 51 72) (end 50 73) (width 0.25) (layer "B.Cu") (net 49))
 (segment (start 45.295489 136.704211) (end 45.295489 138.294511) (width 0.25) (layer "B.Cu") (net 49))
 (segment (start 45.295489 138.294511) (end 43.88 139.71) (width 0.25) (layer "B.Cu") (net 49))
 (segment (start 49.343889 124.343889) (end 49.343889 125.143657) (width 0.25) (layer "B.Cu") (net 49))
 (segment (start 47.835489 122.835489) (end 49.343889 124.343889) (width 0.25) (layer "B.Cu") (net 49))
 (segment (start 47.835489 81.164511) (end 47.835489 122.835489) (width 0.25) (layer "B.Cu") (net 49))
 (segment (start 51.292911 126.336343) (end 51.292911 130.706789) (width 0.25) (layer "B.Cu") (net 49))
 (segment (start 51.292911 130.706789) (end 45.295489 136.704211) (width 0.25) (layer "B.Cu") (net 49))
 (segment (start 49.343889 125.143657) (end 49.914743 125.714511) (width 0.25) (layer "B.Cu") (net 49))
 (segment (start 49.914743 125.714511) (end 50.671079 125.714511) (width 0.25) (layer "B.Cu") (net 49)))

